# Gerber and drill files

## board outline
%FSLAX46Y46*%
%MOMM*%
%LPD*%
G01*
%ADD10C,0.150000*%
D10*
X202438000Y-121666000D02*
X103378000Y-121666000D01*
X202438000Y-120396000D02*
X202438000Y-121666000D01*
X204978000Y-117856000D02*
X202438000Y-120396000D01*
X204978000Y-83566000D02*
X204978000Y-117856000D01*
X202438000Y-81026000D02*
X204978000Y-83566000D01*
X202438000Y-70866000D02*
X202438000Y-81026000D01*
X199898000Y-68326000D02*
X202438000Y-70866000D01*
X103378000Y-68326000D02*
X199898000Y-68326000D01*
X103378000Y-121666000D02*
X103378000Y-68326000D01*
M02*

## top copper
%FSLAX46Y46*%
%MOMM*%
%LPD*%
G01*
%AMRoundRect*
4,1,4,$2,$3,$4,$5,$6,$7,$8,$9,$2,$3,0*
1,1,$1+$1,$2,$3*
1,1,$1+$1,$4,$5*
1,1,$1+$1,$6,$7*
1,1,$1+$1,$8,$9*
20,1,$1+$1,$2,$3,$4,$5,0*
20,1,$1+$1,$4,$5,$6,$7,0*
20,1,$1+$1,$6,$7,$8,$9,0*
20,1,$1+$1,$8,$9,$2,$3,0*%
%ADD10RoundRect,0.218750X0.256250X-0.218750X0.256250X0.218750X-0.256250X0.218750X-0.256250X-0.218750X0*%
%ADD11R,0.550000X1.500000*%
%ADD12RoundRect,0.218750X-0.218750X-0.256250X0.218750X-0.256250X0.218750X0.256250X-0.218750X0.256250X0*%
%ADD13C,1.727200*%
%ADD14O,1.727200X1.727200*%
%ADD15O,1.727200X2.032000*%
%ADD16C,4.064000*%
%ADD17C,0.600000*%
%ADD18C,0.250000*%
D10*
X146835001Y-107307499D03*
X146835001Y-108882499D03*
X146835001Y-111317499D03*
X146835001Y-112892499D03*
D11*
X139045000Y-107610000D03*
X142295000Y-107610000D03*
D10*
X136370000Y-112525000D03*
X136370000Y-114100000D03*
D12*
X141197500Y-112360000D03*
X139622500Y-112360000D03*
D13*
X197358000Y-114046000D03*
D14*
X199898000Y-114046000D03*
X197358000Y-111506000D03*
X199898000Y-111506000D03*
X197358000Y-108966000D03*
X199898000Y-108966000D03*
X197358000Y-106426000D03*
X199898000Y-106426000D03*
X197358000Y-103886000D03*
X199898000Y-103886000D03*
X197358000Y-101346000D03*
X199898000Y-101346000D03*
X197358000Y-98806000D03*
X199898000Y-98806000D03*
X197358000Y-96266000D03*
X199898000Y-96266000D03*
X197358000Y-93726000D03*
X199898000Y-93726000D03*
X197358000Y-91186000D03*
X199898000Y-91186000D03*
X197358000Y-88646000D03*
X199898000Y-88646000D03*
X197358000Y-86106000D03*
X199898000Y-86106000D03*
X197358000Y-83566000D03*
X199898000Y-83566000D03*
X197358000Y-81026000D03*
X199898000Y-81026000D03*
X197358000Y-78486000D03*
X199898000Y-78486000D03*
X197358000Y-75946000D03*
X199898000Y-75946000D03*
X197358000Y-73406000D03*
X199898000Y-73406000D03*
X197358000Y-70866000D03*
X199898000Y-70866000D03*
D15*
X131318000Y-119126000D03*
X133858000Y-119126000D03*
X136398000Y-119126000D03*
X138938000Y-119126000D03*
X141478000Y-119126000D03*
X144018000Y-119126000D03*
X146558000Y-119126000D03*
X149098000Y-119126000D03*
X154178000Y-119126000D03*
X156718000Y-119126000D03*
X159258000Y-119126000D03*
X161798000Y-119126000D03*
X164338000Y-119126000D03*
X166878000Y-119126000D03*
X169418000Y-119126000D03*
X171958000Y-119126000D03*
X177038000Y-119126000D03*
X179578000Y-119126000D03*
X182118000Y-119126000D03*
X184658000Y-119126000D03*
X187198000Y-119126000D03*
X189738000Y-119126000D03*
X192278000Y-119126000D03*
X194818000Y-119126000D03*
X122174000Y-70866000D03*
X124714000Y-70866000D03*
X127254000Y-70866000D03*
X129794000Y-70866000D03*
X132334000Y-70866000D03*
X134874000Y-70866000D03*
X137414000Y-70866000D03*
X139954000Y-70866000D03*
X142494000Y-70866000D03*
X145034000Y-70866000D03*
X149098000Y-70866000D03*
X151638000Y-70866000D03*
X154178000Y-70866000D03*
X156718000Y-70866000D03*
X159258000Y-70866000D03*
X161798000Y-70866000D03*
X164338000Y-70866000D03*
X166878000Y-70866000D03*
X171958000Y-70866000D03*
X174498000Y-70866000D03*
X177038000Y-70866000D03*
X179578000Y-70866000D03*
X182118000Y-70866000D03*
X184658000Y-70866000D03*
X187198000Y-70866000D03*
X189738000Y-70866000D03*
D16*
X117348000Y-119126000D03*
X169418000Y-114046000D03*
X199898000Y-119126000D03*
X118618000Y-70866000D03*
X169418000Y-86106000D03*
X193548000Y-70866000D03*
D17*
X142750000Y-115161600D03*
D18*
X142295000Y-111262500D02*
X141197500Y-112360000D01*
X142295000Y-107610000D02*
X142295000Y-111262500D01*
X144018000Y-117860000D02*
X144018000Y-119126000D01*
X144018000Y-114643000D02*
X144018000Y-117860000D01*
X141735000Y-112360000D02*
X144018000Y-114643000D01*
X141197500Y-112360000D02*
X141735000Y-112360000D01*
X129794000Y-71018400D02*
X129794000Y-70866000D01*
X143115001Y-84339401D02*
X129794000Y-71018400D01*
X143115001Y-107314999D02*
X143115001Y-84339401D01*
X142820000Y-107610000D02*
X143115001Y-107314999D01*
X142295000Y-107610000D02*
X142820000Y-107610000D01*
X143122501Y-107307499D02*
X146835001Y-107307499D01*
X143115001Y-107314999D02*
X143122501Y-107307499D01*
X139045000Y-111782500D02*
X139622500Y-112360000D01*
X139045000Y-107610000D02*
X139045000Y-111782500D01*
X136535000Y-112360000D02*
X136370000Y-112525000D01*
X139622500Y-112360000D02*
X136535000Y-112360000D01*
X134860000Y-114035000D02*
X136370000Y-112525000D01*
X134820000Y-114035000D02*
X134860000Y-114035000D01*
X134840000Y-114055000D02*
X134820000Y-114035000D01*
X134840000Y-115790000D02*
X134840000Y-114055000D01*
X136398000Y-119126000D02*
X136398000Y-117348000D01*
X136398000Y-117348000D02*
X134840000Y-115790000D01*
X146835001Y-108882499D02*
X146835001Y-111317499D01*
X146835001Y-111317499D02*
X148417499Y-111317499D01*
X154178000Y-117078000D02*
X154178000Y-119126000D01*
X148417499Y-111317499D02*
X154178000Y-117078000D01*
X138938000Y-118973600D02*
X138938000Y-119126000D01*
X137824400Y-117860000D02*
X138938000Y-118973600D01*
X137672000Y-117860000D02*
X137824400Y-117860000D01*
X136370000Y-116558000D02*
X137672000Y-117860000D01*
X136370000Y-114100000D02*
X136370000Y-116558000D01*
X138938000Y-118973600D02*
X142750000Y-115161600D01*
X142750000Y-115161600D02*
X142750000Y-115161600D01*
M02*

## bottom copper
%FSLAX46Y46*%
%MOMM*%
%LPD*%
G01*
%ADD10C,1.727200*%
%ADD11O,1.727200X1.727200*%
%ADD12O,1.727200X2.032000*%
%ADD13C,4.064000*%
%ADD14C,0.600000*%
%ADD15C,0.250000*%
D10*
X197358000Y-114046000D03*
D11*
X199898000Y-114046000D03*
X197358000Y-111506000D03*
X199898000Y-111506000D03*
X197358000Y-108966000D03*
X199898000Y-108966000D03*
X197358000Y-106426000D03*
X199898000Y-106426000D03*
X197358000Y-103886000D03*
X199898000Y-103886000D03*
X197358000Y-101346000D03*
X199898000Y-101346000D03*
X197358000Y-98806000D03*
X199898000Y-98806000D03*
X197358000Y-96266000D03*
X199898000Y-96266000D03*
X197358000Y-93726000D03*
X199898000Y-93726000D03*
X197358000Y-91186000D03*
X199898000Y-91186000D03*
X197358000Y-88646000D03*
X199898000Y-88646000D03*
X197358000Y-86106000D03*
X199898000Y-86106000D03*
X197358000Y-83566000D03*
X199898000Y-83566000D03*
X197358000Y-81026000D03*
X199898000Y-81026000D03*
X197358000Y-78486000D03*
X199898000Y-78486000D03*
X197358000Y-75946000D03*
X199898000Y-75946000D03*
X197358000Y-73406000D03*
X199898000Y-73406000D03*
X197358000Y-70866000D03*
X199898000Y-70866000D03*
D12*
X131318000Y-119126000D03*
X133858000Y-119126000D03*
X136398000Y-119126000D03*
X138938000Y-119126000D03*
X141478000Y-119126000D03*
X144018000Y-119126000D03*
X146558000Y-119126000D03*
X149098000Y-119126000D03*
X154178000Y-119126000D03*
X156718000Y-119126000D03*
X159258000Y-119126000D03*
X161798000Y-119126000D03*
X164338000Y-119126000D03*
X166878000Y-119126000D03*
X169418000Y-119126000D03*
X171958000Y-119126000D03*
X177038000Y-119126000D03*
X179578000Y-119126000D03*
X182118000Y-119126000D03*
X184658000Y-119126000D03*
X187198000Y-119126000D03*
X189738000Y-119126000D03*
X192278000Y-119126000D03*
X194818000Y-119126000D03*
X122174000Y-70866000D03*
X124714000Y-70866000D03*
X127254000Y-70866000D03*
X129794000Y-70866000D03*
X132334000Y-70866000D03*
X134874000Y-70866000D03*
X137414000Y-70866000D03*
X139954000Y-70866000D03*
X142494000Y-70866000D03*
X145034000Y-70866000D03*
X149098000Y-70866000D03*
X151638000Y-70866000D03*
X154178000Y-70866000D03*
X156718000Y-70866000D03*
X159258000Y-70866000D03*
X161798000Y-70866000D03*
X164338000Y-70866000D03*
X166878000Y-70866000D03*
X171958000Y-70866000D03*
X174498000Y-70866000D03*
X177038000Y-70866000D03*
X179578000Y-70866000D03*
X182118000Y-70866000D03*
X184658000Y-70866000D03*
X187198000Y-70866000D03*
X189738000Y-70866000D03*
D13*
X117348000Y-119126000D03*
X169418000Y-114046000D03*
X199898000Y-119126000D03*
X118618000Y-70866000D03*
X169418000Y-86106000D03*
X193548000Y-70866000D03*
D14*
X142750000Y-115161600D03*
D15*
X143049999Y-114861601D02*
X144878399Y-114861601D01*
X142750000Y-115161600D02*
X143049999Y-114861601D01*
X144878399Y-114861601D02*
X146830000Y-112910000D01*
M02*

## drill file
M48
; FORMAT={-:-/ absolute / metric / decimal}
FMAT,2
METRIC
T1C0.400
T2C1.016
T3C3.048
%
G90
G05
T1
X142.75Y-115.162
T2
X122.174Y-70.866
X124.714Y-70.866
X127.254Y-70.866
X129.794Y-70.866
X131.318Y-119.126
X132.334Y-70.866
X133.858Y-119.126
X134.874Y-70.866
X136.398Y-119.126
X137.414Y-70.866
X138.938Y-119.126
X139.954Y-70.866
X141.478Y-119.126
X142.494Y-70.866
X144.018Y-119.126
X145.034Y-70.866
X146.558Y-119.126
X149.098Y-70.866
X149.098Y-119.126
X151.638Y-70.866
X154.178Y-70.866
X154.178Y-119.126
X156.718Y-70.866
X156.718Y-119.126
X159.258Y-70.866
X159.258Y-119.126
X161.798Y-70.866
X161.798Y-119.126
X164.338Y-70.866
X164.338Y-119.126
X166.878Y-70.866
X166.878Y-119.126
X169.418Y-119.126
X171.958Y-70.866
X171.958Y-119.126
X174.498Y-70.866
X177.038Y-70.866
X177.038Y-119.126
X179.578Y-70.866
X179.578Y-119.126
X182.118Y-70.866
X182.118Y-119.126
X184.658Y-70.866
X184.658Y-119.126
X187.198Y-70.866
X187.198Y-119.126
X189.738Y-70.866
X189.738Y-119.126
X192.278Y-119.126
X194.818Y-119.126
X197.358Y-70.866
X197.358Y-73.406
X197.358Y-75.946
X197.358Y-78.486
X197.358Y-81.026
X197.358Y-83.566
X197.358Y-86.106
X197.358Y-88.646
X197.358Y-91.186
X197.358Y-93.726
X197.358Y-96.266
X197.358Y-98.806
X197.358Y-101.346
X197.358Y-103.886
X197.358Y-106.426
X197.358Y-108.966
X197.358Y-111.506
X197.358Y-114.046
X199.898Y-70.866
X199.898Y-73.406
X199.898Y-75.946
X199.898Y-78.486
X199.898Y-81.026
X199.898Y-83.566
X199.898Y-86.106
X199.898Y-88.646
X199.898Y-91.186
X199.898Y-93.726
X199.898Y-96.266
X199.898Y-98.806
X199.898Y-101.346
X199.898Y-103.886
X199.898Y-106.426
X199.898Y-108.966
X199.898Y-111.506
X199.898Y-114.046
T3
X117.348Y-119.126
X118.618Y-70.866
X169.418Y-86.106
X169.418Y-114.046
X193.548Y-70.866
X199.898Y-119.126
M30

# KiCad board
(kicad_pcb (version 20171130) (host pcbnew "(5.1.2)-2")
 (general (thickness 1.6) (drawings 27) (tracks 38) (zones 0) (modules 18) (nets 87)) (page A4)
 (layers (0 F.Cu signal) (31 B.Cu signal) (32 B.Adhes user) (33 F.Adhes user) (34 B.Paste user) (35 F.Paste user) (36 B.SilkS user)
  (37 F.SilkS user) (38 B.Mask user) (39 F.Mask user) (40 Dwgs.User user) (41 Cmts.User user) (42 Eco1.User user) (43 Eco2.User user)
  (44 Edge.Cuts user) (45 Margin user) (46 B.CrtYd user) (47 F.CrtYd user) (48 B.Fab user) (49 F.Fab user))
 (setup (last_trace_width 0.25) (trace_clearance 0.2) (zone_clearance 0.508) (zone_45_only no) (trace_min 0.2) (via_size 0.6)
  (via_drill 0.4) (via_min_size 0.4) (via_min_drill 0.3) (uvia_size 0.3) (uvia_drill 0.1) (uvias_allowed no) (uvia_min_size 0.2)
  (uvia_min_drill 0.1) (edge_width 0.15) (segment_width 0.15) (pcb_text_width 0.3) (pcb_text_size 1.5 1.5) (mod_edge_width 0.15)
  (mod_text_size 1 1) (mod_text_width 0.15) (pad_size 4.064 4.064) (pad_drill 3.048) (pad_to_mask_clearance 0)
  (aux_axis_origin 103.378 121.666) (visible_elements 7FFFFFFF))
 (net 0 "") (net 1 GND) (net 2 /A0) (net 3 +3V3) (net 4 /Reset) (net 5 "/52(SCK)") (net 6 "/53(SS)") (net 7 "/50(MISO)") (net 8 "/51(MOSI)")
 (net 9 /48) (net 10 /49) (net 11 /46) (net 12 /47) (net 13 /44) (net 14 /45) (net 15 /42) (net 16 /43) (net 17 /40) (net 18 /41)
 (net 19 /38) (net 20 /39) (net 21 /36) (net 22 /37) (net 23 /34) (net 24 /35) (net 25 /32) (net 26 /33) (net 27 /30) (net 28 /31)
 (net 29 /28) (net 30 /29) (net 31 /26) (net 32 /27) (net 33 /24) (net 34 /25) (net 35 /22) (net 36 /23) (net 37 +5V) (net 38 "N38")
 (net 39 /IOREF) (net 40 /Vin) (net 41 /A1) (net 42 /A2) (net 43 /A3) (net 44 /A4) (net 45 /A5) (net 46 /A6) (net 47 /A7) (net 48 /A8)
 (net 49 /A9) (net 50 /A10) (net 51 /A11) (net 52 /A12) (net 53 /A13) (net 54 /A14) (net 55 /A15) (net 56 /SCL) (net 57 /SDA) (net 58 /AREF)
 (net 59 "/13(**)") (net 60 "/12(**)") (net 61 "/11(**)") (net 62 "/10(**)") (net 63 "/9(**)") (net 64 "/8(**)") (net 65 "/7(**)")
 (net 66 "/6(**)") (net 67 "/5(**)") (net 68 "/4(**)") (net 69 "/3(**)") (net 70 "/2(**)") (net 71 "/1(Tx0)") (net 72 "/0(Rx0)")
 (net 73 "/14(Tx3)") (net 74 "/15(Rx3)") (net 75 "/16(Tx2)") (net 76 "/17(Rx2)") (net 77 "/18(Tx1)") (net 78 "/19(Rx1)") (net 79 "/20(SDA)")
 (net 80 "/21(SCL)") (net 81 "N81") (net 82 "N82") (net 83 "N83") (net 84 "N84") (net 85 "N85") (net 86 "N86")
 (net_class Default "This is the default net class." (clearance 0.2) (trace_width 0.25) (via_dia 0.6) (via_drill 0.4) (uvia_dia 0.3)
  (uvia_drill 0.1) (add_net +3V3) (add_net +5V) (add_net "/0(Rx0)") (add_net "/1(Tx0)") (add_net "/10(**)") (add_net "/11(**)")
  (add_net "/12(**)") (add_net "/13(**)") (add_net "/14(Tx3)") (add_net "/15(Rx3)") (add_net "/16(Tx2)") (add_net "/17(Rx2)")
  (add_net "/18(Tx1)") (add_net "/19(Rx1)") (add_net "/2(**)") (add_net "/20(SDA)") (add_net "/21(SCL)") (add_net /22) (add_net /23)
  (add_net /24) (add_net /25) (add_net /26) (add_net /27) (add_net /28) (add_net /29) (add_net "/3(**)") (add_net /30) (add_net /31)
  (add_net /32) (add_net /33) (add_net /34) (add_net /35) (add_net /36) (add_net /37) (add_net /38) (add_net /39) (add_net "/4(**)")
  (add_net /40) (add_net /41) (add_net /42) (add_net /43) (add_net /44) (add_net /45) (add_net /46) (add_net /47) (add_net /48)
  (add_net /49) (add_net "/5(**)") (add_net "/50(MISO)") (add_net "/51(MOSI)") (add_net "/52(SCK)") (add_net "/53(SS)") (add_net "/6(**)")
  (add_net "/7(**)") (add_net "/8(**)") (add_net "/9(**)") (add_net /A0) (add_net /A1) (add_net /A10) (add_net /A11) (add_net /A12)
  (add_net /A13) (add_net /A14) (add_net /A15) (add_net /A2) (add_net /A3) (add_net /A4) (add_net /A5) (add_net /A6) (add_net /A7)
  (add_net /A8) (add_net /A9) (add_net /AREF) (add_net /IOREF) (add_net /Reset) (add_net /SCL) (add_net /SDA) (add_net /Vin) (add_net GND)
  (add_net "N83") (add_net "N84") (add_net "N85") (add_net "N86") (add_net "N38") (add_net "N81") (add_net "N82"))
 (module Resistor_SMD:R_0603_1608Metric (layer F.Cu) (at 146.835001 108.094999 90)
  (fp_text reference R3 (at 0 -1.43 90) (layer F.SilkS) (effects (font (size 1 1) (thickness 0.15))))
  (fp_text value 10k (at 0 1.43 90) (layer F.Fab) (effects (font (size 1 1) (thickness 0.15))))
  (pad 2 smd roundrect (at 0.7875 0 90) (size 0.875 0.95) (layers F.Cu F.Paste F.Mask) (roundrect_rratio 0.25) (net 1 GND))
  (pad 1 smd roundrect (at -0.7875 0 90) (size 0.875 0.95) (layers F.Cu F.Paste F.Mask) (roundrect_rratio 0.25) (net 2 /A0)))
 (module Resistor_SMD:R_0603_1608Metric (layer F.Cu) (at 146.835001 112.104999 90)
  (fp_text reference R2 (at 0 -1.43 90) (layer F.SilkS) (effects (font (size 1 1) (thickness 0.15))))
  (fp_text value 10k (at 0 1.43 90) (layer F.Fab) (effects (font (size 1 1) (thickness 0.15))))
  (pad 2 smd roundrect (at 0.7875 0 90) (size 0.875 0.95) (layers F.Cu F.Paste F.Mask) (roundrect_rratio 0.25) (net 2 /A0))
  (pad 1 smd roundrect (at -0.7875 0 90) (size 0.875 0.95) (layers F.Cu F.Paste F.Mask) (roundrect_rratio 0.25) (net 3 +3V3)))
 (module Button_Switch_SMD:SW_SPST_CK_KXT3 (layer F.Cu) (at 140.67 107.61 180)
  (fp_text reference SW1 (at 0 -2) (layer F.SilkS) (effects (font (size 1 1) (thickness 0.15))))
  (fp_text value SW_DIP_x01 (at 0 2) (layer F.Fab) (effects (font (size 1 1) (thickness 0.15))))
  (pad 2 smd rect (at 1.625 0 180) (size 0.55 1.5) (layers F.Cu F.Paste F.Mask) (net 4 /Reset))
  (pad 1 smd rect (at -1.625 0 180) (size 0.55 1.5) (layers F.Cu F.Paste F.Mask) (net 1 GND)))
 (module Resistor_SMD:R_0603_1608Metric (layer F.Cu) (at 136.37 113.3125 90)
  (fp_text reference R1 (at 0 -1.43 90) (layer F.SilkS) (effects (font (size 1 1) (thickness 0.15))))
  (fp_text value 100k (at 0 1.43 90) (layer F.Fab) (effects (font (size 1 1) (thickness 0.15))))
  (pad 2 smd roundrect (at 0.7875 0 90) (size 0.875 0.95) (layers F.Cu F.Paste F.Mask) (roundrect_rratio 0.25) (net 4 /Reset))
  (pad 1 smd roundrect (at -0.7875 0 90) (size 0.875 0.95) (layers F.Cu F.Paste F.Mask) (roundrect_rratio 0.25) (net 3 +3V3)))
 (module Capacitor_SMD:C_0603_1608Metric (layer F.Cu) (at 140.41 112.36)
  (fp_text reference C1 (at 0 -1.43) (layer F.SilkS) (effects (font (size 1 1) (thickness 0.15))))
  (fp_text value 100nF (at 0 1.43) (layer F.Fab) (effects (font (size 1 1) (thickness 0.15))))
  (pad 2 smd roundrect (at 0.7875 0) (size 0.875 0.95) (layers F.Cu F.Paste F.Mask) (roundrect_rratio 0.25) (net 1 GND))
  (pad 1 smd roundrect (at -0.7875 0) (size 0.875 0.95) (layers F.Cu F.Paste F.Mask) (roundrect_rratio 0.25) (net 4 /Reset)))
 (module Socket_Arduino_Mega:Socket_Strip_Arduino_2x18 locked (layer F.Cu) (at 197.358 114.046 90)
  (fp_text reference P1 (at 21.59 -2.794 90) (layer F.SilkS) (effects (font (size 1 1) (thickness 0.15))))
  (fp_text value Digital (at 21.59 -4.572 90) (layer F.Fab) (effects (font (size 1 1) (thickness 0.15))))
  (pad 1 thru_hole circle (at 0 0 90) (size 1.7272 1.7272) (drill 1.016) (layers *.Cu *.Mask F.SilkS) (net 1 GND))
  (pad 2 thru_hole oval (at 0 2.54 90) (size 1.7272 1.7272) (drill 1.016) (layers *.Cu *.Mask F.SilkS) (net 1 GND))
  (pad 3 thru_hole oval (at 2.54 0 90) (size 1.7272 1.7272) (drill 1.016) (layers *.Cu *.Mask F.SilkS) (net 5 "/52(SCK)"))
  (pad 4 thru_hole oval (at 2.54 2.54 90) (size 1.7272 1.7272) (drill 1.016) (layers *.Cu *.Mask F.SilkS) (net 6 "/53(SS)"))
  (pad 5 thru_hole oval (at 5.08 0 90) (size 1.7272 1.7272) (drill 1.016) (layers *.Cu *.Mask F.SilkS) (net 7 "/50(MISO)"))
  (pad 6 thru_hole oval (at 5.08 2.54 90) (size 1.7272 1.7272) (drill 1.016) (layers *.Cu *.Mask F.SilkS) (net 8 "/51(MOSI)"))
  (pad 7 thru_hole oval (at 7.62 0 90) (size 1.7272 1.7272) (drill 1.016) (layers *.Cu *.Mask F.SilkS) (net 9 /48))
  (pad 8 thru_hole oval (at 7.62 2.54 90) (size 1.7272 1.7272) (drill 1.016) (layers *.Cu *.Mask F.SilkS) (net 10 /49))
  (pad 9 thru_hole oval (at 10.16 0 90) (size 1.7272 1.7272) (drill 1.016) (layers *.Cu *.Mask F.SilkS) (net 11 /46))
  (pad 10 thru_hole oval (at 10.16 2.54 90) (size 1.7272 1.7272) (drill 1.016) (layers *.Cu *.Mask F.SilkS) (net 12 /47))
  (pad 11 thru_hole oval (at 12.7 0 90) (size 1.7272 1.7272) (drill 1.016) (layers *.Cu *.Mask F.SilkS) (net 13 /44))
  (pad 12 thru_hole oval (at 12.7 2.54 90) (size 1.7272 1.7272) (drill 1.016) (layers *.Cu *.Mask F.SilkS) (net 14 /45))
  (pad 13 thru_hole oval (at 15.24 0 90) (size 1.7272 1.7272) (drill 1.016) (layers *.Cu *.Mask F.SilkS) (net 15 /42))
  (pad 14 thru_hole oval (at 15.24 2.54 90) (size 1.7272 1.7272) (drill 1.016) (layers *.Cu *.Mask F.SilkS) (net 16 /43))
  (pad 15 thru_hole oval (at 17.78 0 90) (size 1.7272 1.7272) (drill 1.016) (layers *.Cu *.Mask F.SilkS) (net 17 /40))
  (pad 16 thru_hole oval (at 17.78 2.54 90) (size 1.7272 1.7272) (drill 1.016) (layers *.Cu *.Mask F.SilkS) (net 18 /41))
  (pad 17 thru_hole oval (at 20.32 0 90) (size 1.7272 1.7272) (drill 1.016) (layers *.Cu *.Mask F.SilkS) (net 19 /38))
  (pad 18 thru_hole oval (at 20.32 2.54 90) (size 1.7272 1.7272) (drill 1.016) (layers *.Cu *.Mask F.SilkS) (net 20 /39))
  (pad 19 thru_hole oval (at 22.86 0 90) (size 1.7272 1.7272) (drill 1.016) (layers *.Cu *.Mask F.SilkS) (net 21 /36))
  (pad 20 thru_hole oval (at 22.86 2.54 90) (size 1.7272 1.7272) (drill 1.016) (layers *.Cu *.Mask F.SilkS) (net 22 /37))
  (pad 21 thru_hole oval (at 25.4 0 90) (size 1.7272 1.7272) (drill 1.016) (layers *.Cu *.Mask F.SilkS) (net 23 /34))
  (pad 22 thru_hole oval (at 25.4 2.54 90) (size 1.7272 1.7272) (drill 1.016) (layers *.Cu *.Mask F.SilkS) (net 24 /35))
  (pad 23 thru_hole oval (at 27.94 0 90) (size 1.7272 1.7272) (drill 1.016) (layers *.Cu *.Mask F.SilkS) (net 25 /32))
  (pad 24 thru_hole oval (at 27.94 2.54 90) (size 1.7272 1.7272) (drill 1.016) (layers *.Cu *.Mask F.SilkS) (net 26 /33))
  (pad 25 thru_hole oval (at 30.48 0 90) (size 1.7272 1.7272) (drill 1.016) (layers *.Cu *.Mask F.SilkS) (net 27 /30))
  (pad 26 thru_hole oval (at 30.48 2.54 90) (size 1.7272 1.7272) (drill 1.016) (layers *.Cu *.Mask F.SilkS) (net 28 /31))
  (pad 27 thru_hole oval (at 33.02 0 90) (size 1.7272 1.7272) (drill 1.016) (layers *.Cu *.Mask F.SilkS) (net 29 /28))
  (pad 28 thru_hole oval (at 33.02 2.54 90) (size 1.7272 1.7272) (drill 1.016) (layers *.Cu *.Mask F.SilkS) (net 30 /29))
  (pad 29 thru_hole oval (at 35.56 0 90) (size 1.7272 1.7272) (drill 1.016) (layers *.Cu *.Mask F.SilkS) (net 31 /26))
  (pad 30 thru_hole oval (at 35.56 2.54 90) (size 1.7272 1.7272) (drill 1.016) (layers *.Cu *.Mask F.SilkS) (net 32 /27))
  (pad 31 thru_hole oval (at 38.1 0 90) (size 1.7272 1.7272) (drill 1.016) (layers *.Cu *.Mask F.SilkS) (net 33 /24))
  (pad 32 thru_hole oval (at 38.1 2.54 90) (size 1.7272 1.7272) (drill 1.016) (layers *.Cu *.Mask F.SilkS) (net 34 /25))
  (pad 33 thru_hole oval (at 40.64 0 90) (size 1.7272 1.7272) (drill 1.016) (layers *.Cu *.Mask F.SilkS) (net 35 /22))
  (pad 34 thru_hole oval (at 40.64 2.54 90) (size 1.7272 1.7272) (drill 1.016) (layers *.Cu *.Mask F.SilkS) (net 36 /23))
  (pad 35 thru_hole oval (at 43.18 0 90) (size 1.7272 1.7272) (drill 1.016) (layers *.Cu *.Mask F.SilkS) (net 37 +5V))
  (pad 36 thru_hole oval (at 43.18 2.54 90) (size 1.7272 1.7272) (drill 1.016) (layers *.Cu *.Mask F.SilkS) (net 37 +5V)))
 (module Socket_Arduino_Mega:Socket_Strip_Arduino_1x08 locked (layer F.Cu) (at 131.318 119.126)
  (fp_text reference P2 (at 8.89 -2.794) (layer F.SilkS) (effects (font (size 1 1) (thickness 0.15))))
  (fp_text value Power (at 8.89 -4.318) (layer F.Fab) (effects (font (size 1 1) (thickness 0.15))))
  (pad 1 thru_hole oval (at 0 0) (size 1.7272 2.032) (drill 1.016) (layers *.Cu *.Mask F.SilkS) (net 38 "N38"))
  (pad 2 thru_hole oval (at 2.54 0) (size 1.7272 2.032) (drill 1.016) (layers *.Cu *.Mask F.SilkS) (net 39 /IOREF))
  (pad 3 thru_hole oval (at 5.08 0) (size 1.7272 2.032) (drill 1.016) (layers *.Cu *.Mask F.SilkS) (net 4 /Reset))
  (pad 4 thru_hole oval (at 7.62 0) (size 1.7272 2.032) (drill 1.016) (layers *.Cu *.Mask F.SilkS) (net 3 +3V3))
  (pad 5 thru_hole oval (at 10.16 0) (size 1.7272 2.032) (drill 1.016) (layers *.Cu *.Mask F.SilkS) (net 37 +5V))
  (pad 6 thru_hole oval (at 12.7 0) (size 1.7272 2.032) (drill 1.016) (layers *.Cu *.Mask F.SilkS) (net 1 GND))
  (pad 7 thru_hole oval (at 15.24 0) (size 1.7272 2.032) (drill 1.016) (layers *.Cu *.Mask F.SilkS) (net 1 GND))
  (pad 8 thru_hole oval (at 17.78 0) (size 1.7272 2.032) (drill 1.016) (layers *.Cu *.Mask F.SilkS) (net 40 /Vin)))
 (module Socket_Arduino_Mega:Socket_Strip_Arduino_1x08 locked (layer F.Cu) (at 154.178 119.126)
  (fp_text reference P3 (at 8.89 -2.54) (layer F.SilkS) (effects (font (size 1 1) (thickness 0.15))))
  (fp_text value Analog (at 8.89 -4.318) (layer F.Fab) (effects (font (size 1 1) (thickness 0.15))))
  (pad 1 thru_hole oval (at 0 0) (size 1.7272 2.032) (drill 1.016) (layers *.Cu *.Mask F.SilkS) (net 2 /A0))
  (pad 2 thru_hole oval (at 2.54 0) (size 1.7272 2.032) (drill 1.016) (layers *.Cu *.Mask F.SilkS) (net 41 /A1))
  (pad 3 thru_hole oval (at 5.08 0) (size 1.7272 2.032) (drill 1.016) (layers *.Cu *.Mask F.SilkS) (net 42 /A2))
  (pad 4 thru_hole oval (at 7.62 0) (size 1.7272 2.032) (drill 1.016) (layers *.Cu *.Mask F.SilkS) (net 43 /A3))
  (pad 5 thru_hole oval (at 10.16 0) (size 1.7272 2.032) (drill 1.016) (layers *.Cu *.Mask F.SilkS) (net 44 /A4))
  (pad 6 thru_hole oval (at 12.7 0) (size 1.7272 2.032) (drill 1.016) (layers *.Cu *.Mask F.SilkS) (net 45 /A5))
  (pad 7 thru_hole oval (at 15.24 0) (size 1.7272 2.032) (drill 1.016) (layers *.Cu *.Mask F.SilkS) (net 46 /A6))
  (pad 8 thru_hole oval (at 17.78 0) (size 1.7272 2.032) (drill 1.016) (layers *.Cu *.Mask F.SilkS) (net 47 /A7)))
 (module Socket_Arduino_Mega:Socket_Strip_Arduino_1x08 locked (layer F.Cu) (at 177.038 119.126)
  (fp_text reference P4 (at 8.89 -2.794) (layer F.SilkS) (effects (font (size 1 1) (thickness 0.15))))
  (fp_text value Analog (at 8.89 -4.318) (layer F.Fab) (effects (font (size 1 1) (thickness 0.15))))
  (pad 1 thru_hole oval (at 0 0) (size 1.7272 2.032) (drill 1.016) (layers *.Cu *.Mask F.SilkS) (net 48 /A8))
  (pad 2 thru_hole oval (at 2.54 0) (size 1.7272 2.032) (drill 1.016) (layers *.Cu *.Mask F.SilkS) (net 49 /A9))
  (pad 3 thru_hole oval (at 5.08 0) (size 1.7272 2.032) (drill 1.016) (layers *.Cu *.Mask F.SilkS) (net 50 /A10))
  (pad 4 thru_hole oval (at 7.62 0) (size 1.7272 2.032) (drill 1.016) (layers *.Cu *.Mask F.SilkS) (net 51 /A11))
  (pad 5 thru_hole oval (at 10.16 0) (size 1.7272 2.032) (drill 1.016) (layers *.Cu *.Mask F.SilkS) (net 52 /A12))
  (pad 6 thru_hole oval (at 12.7 0) (size 1.7272 2.032) (drill 1.016) (layers *.Cu *.Mask F.SilkS) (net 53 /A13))
  (pad 7 thru_hole oval (at 15.24 0) (size 1.7272 2.032) (drill 1.016) (layers *.Cu *.Mask F.SilkS) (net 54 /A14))
  (pad 8 thru_hole oval (at 17.78 0) (size 1.7272 2.032) (drill 1.016) (layers *.Cu *.Mask F.SilkS) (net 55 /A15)))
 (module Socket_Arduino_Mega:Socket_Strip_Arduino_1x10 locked (layer F.Cu) (at 122.174 70.866)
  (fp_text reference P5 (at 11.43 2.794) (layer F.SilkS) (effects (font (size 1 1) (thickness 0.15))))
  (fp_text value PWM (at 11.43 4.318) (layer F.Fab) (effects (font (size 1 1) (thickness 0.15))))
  (pad 1 thru_hole oval (at 0 0) (size 1.7272 2.032) (drill 1.016) (layers *.Cu *.Mask F.SilkS) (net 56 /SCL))
  (pad 2 thru_hole oval (at 2.54 0) (size 1.7272 2.032) (drill 1.016) (layers *.Cu *.Mask F.SilkS) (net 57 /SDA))
  (pad 3 thru_hole oval (at 5.08 0) (size 1.7272 2.032) (drill 1.016) (layers *.Cu *.Mask F.SilkS) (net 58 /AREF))
  (pad 4 thru_hole oval (at 7.62 0) (size 1.7272 2.032) (drill 1.016) (layers *.Cu *.Mask F.SilkS) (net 1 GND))
  (pad 5 thru_hole oval (at 10.16 0) (size 1.7272 2.032) (drill 1.016) (layers *.Cu *.Mask F.SilkS) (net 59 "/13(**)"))
  (pad 6 thru_hole oval (at 12.7 0) (size 1.7272 2.032) (drill 1.016) (layers *.Cu *.Mask F.SilkS) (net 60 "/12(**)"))
  (pad 7 thru_hole oval (at 15.24 0) (size 1.7272 2.032) (drill 1.016) (layers *.Cu *.Mask F.SilkS) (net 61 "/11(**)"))
  (pad 8 thru_hole oval (at 17.78 0) (size 1.7272 2.032) (drill 1.016) (layers *.Cu *.Mask F.SilkS) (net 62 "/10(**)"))
  (pad 9 thru_hole oval (at 20.32 0) (size 1.7272 2.032) (drill 1.016) (layers *.Cu *.Mask F.SilkS) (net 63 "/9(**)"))
  (pad 10 thru_hole oval (at 22.86 0) (size 1.7272 2.032) (drill 1.016) (layers *.Cu *.Mask F.SilkS) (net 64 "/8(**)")))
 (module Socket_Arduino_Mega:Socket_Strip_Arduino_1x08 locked (layer F.Cu) (at 149.098 70.866)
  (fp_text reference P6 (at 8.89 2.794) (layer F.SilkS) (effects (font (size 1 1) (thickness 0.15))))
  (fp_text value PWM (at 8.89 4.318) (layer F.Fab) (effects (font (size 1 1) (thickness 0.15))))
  (pad 1 thru_hole oval (at 0 0) (size 1.7272 2.032) (drill 1.016) (layers *.Cu *.Mask F.SilkS) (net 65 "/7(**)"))
  (pad 2 thru_hole oval (at 2.54 0) (size 1.7272 2.032) (drill 1.016) (layers *.Cu *.Mask F.SilkS) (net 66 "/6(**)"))
  (pad 3 thru_hole oval (at 5.08 0) (size 1.7272 2.032) (drill 1.016) (layers *.Cu *.Mask F.SilkS) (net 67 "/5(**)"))
  (pad 4 thru_hole oval (at 7.62 0) (size 1.7272 2.032) (drill 1.016) (layers *.Cu *.Mask F.SilkS) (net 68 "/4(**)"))
  (pad 5 thru_hole oval (at 10.16 0) (size 1.7272 2.032) (drill 1.016) (layers *.Cu *.Mask F.SilkS) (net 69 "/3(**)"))
  (pad 6 thru_hole oval (at 12.7 0) (size 1.7272 2.032) (drill 1.016) (layers *.Cu *.Mask F.SilkS) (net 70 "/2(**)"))
  (pad 7 thru_hole oval (at 15.24 0) (size 1.7272 2.032) (drill 1.016) (layers *.Cu *.Mask F.SilkS) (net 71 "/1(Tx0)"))
  (pad 8 thru_hole oval (at 17.78 0) (size 1.7272 2.032) (drill 1.016) (layers *.Cu *.Mask F.SilkS) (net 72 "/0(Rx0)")))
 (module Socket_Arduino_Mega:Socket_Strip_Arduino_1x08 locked (layer F.Cu) (at 171.958 70.866)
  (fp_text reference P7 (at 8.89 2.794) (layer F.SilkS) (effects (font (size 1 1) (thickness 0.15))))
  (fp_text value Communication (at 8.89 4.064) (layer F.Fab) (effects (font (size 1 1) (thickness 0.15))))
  (pad 1 thru_hole oval (at 0 0) (size 1.7272 2.032) (drill 1.016) (layers *.Cu *.Mask F.SilkS) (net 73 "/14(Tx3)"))
  (pad 2 thru_hole oval (at 2.54 0) (size 1.7272 2.032) (drill 1.016) (layers *.Cu *.Mask F.SilkS) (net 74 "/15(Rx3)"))
  (pad 3 thru_hole oval (at 5.08 0) (size 1.7272 2.032) (drill 1.016) (layers *.Cu *.Mask F.SilkS) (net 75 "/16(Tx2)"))
  (pad 4 thru_hole oval (at 7.62 0) (size 1.7272 2.032) (drill 1.016) (layers *.Cu *.Mask F.SilkS) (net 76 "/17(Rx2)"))
  (pad 5 thru_hole oval (at 10.16 0) (size 1.7272 2.032) (drill 1.016) (layers *.Cu *.Mask F.SilkS) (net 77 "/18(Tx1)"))
  (pad 6 thru_hole oval (at 12.7 0) (size 1.7272 2.032) (drill 1.016) (layers *.Cu *.Mask F.SilkS) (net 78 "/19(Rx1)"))
  (pad 7 thru_hole oval (at 15.24 0) (size 1.7272 2.032) (drill 1.016) (layers *.Cu *.Mask F.SilkS) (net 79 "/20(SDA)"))
  (pad 8 thru_hole oval (at 17.78 0) (size 1.7272 2.032) (drill 1.016) (layers *.Cu *.Mask F.SilkS) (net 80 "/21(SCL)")))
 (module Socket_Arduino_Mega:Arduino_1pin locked (layer F.Cu) (at 117.348 119.126)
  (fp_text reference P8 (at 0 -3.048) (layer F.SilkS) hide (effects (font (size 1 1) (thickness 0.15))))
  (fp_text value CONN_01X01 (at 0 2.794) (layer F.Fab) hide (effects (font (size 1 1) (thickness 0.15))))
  (pad 1 thru_hole circle (at 0 0) (size 4.064 4.064) (drill 3.048) (layers *.Cu *.Mask F.SilkS) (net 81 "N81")))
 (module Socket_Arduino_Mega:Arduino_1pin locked (layer F.Cu) (at 169.418 114.046)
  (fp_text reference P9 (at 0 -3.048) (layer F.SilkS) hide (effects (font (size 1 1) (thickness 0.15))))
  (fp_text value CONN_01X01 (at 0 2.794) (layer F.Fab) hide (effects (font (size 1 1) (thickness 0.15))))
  (pad 1 thru_hole circle (at 0 0) (size 4.064 4.064) (drill 3.048) (layers *.Cu *.Mask F.SilkS) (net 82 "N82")))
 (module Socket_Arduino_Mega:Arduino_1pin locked (layer F.Cu) (at 199.898 119.126)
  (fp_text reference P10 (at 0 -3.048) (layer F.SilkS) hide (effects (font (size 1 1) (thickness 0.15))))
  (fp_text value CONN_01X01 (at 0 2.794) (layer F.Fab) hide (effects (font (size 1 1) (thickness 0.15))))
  (pad 1 thru_hole circle (at 0 0) (size 4.064 4.064) (drill 3.048) (layers *.Cu *.Mask F.SilkS) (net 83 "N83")))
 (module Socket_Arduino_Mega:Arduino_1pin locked (layer F.Cu) (at 118.618 70.866)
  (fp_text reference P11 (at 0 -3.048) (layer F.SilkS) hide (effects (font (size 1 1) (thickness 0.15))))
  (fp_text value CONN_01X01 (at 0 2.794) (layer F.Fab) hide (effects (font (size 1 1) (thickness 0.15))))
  (pad 1 thru_hole circle (at 0 0) (size 4.064 4.064) (drill 3.048) (layers *.Cu *.Mask F.SilkS) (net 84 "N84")))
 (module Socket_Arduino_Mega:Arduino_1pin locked (layer F.Cu) (at 169.418 86.106)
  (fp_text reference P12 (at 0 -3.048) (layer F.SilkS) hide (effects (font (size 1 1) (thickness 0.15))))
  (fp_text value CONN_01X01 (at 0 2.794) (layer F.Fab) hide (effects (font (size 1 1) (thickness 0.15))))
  (pad 1 thru_hole circle (at 0 0) (size 4.064 4.064) (drill 3.048) (layers *.Cu *.Mask F.SilkS) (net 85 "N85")))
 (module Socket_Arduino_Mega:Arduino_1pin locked (layer F.Cu) (at 193.548 70.866)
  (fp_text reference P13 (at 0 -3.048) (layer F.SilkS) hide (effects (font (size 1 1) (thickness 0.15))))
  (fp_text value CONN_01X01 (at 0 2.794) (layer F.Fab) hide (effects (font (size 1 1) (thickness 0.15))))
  (pad 1 thru_hole circle (at 0 0) (size 4.064 4.064) (drill 3.048) (layers *.Cu *.Mask F.SilkS) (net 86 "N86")))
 (gr_line (start 202.438 121.666) (end 103.378 121.666) (angle 90) (layer Edge.Cuts) (width 0.15))
 (gr_line (start 202.438 120.396) (end 202.438 121.666) (angle 90) (layer Edge.Cuts) (width 0.15))
 (gr_line (start 204.978 117.856) (end 202.438 120.396) (angle 90) (layer Edge.Cuts) (width 0.15))
 (gr_line (start 204.978 83.566) (end 204.978 117.856) (angle 90) (layer Edge.Cuts) (width 0.15))
 (gr_line (start 202.438 81.026) (end 204.978 83.566) (angle 90) (layer Edge.Cuts) (width 0.15))
 (gr_line (start 202.438 70.866) (end 202.438 81.026) (angle 90) (layer Edge.Cuts) (width 0.15))
 (gr_line (start 199.898 68.326) (end 202.438 70.866) (angle 90) (layer Edge.Cuts) (width 0.15))
 (gr_line (start 103.378 68.326) (end 199.898 68.326) (angle 90) (layer Edge.Cuts) (width 0.15))
 (gr_line (start 103.378 121.666) (end 103.378 68.326) (angle 90) (layer Edge.Cuts) (width 0.15))
 (segment (start 142.295 111.2625) (end 141.1975 112.36) (width 0.25) (layer F.Cu) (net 1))
 (segment (start 142.295 107.61) (end 142.295 111.2625) (width 0.25) (layer F.Cu) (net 1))
 (segment (start 144.018 117.86) (end 144.018 119.126) (width 0.25) (layer F.Cu) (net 1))
 (segment (start 144.018 114.643) (end 144.018 117.86) (width 0.25) (layer F.Cu) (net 1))
 (segment (start 141.735 112.36) (end 144.018 114.643) (width 0.25) (layer F.Cu) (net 1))
 (segment (start 141.1975 112.36) (end 141.735 112.36) (width 0.25) (layer F.Cu) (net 1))
 (segment (start 129.794 71.0184) (end 129.794 70.866) (width 0.25) (layer F.Cu) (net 1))
 (segment (start 143.115001 84.339401) (end 129.794 71.0184) (width 0.25) (layer F.Cu) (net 1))
 (segment (start 143.115001 107.314999) (end 143.115001 84.339401) (width 0.25) (layer F.Cu) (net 1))
 (segment (start 142.82 107.61) (end 143.115001 107.314999) (width 0.25) (layer F.Cu) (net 1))
 (segment (start 142.295 107.61) (end 142.82 107.61) (width 0.25) (layer F.Cu) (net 1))
 (segment (start 143.122501 107.307499) (end 146.835001 107.307499) (width 0.25) (layer F.Cu) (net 1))
 (segment (start 143.115001 107.314999) (end 143.122501 107.307499) (width 0.25) (layer F.Cu) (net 1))
 (segment (start 139.045 111.7825) (end 139.6225 112.36) (width 0.25) (layer F.Cu) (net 4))
 (segment (start 139.045 107.61) (end 139.045 111.7825) (width 0.25) (layer F.Cu) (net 4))
 (segment (start 136.535 112.36) (end 136.37 112.525) (width 0.25) (layer F.Cu) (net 4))
 (segment (start 139.6225 112.36) (end 136.535 112.36) (width 0.25) (layer F.Cu) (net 4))
 (segment (start 134.86 114.035) (end 136.37 112.525) (width 0.25) (layer F.Cu) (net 4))
 (segment (start 134.82 114.035) (end 134.86 114.035) (width 0.25) (layer F.Cu) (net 4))
 (segment (start 134.84 114.055) (end 134.82 114.035) (width 0.25) (layer F.Cu) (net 4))
 (segment (start 134.84 115.79) (end 134.84 114.055) (width 0.25) (layer F.Cu) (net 4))
 (segment (start 136.398 119.126) (end 136.398 117.348) (width 0.25) (layer F.Cu) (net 4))
 (segment (start 136.398 117.348) (end 134.84 115.79) (width 0.25) (layer F.Cu) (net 4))
 (segment (start 146.835001 108.882499) (end 146.835001 111.317499) (width 0.25) (layer F.Cu) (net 2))
 (segment (start 146.835001 111.317499) (end 148.417499 111.317499) (width 0.25) (layer F.Cu) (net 2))
 (segment (start 154.178 117.078) (end 154.178 119.126) (width 0.25) (layer F.Cu) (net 2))
 (segment (start 148.417499 111.317499) (end 154.178 117.078) (width 0.25) (layer F.Cu) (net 2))
 (segment (start 138.938 118.9736) (end 138.938 119.126) (width 0.25) (layer F.Cu) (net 3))
 (segment (start 137.8244 117.86) (end 138.938 118.9736) (width 0.25) (layer F.Cu) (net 3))
 (segment (start 137.672 117.86) (end 137.8244 117.86) (width 0.25) (layer F.Cu) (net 3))
 (segment (start 136.37 116.558) (end 137.672 117.86) (width 0.25) (layer F.Cu) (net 3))
 (segment (start 136.37 114.1) (end 136.37 116.558) (width 0.25) (layer F.Cu) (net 3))
 (segment (start 138.938 118.9736) (end 142.75 115.1616) (width 0.25) (layer F.Cu) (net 3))
 (segment (start 142.75 115.1616) (end 142.75 115.1616) (width 0.25) (layer F.Cu) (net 3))
 (via (at 142.75 115.1616) (size 0.6) (drill 0.4) (layers F.Cu B.Cu) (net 3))
 (segment (start 143.049999 114.861601) (end 144.878399 114.861601) (width 0.25) (layer B.Cu) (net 3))
 (segment (start 142.75 115.1616) (end 143.049999 114.861601) (width 0.25) (layer B.Cu) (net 3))
 (segment (start 144.878399 114.861601) (end 146.83 112.91) (width 0.25) (layer B.Cu) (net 3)))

